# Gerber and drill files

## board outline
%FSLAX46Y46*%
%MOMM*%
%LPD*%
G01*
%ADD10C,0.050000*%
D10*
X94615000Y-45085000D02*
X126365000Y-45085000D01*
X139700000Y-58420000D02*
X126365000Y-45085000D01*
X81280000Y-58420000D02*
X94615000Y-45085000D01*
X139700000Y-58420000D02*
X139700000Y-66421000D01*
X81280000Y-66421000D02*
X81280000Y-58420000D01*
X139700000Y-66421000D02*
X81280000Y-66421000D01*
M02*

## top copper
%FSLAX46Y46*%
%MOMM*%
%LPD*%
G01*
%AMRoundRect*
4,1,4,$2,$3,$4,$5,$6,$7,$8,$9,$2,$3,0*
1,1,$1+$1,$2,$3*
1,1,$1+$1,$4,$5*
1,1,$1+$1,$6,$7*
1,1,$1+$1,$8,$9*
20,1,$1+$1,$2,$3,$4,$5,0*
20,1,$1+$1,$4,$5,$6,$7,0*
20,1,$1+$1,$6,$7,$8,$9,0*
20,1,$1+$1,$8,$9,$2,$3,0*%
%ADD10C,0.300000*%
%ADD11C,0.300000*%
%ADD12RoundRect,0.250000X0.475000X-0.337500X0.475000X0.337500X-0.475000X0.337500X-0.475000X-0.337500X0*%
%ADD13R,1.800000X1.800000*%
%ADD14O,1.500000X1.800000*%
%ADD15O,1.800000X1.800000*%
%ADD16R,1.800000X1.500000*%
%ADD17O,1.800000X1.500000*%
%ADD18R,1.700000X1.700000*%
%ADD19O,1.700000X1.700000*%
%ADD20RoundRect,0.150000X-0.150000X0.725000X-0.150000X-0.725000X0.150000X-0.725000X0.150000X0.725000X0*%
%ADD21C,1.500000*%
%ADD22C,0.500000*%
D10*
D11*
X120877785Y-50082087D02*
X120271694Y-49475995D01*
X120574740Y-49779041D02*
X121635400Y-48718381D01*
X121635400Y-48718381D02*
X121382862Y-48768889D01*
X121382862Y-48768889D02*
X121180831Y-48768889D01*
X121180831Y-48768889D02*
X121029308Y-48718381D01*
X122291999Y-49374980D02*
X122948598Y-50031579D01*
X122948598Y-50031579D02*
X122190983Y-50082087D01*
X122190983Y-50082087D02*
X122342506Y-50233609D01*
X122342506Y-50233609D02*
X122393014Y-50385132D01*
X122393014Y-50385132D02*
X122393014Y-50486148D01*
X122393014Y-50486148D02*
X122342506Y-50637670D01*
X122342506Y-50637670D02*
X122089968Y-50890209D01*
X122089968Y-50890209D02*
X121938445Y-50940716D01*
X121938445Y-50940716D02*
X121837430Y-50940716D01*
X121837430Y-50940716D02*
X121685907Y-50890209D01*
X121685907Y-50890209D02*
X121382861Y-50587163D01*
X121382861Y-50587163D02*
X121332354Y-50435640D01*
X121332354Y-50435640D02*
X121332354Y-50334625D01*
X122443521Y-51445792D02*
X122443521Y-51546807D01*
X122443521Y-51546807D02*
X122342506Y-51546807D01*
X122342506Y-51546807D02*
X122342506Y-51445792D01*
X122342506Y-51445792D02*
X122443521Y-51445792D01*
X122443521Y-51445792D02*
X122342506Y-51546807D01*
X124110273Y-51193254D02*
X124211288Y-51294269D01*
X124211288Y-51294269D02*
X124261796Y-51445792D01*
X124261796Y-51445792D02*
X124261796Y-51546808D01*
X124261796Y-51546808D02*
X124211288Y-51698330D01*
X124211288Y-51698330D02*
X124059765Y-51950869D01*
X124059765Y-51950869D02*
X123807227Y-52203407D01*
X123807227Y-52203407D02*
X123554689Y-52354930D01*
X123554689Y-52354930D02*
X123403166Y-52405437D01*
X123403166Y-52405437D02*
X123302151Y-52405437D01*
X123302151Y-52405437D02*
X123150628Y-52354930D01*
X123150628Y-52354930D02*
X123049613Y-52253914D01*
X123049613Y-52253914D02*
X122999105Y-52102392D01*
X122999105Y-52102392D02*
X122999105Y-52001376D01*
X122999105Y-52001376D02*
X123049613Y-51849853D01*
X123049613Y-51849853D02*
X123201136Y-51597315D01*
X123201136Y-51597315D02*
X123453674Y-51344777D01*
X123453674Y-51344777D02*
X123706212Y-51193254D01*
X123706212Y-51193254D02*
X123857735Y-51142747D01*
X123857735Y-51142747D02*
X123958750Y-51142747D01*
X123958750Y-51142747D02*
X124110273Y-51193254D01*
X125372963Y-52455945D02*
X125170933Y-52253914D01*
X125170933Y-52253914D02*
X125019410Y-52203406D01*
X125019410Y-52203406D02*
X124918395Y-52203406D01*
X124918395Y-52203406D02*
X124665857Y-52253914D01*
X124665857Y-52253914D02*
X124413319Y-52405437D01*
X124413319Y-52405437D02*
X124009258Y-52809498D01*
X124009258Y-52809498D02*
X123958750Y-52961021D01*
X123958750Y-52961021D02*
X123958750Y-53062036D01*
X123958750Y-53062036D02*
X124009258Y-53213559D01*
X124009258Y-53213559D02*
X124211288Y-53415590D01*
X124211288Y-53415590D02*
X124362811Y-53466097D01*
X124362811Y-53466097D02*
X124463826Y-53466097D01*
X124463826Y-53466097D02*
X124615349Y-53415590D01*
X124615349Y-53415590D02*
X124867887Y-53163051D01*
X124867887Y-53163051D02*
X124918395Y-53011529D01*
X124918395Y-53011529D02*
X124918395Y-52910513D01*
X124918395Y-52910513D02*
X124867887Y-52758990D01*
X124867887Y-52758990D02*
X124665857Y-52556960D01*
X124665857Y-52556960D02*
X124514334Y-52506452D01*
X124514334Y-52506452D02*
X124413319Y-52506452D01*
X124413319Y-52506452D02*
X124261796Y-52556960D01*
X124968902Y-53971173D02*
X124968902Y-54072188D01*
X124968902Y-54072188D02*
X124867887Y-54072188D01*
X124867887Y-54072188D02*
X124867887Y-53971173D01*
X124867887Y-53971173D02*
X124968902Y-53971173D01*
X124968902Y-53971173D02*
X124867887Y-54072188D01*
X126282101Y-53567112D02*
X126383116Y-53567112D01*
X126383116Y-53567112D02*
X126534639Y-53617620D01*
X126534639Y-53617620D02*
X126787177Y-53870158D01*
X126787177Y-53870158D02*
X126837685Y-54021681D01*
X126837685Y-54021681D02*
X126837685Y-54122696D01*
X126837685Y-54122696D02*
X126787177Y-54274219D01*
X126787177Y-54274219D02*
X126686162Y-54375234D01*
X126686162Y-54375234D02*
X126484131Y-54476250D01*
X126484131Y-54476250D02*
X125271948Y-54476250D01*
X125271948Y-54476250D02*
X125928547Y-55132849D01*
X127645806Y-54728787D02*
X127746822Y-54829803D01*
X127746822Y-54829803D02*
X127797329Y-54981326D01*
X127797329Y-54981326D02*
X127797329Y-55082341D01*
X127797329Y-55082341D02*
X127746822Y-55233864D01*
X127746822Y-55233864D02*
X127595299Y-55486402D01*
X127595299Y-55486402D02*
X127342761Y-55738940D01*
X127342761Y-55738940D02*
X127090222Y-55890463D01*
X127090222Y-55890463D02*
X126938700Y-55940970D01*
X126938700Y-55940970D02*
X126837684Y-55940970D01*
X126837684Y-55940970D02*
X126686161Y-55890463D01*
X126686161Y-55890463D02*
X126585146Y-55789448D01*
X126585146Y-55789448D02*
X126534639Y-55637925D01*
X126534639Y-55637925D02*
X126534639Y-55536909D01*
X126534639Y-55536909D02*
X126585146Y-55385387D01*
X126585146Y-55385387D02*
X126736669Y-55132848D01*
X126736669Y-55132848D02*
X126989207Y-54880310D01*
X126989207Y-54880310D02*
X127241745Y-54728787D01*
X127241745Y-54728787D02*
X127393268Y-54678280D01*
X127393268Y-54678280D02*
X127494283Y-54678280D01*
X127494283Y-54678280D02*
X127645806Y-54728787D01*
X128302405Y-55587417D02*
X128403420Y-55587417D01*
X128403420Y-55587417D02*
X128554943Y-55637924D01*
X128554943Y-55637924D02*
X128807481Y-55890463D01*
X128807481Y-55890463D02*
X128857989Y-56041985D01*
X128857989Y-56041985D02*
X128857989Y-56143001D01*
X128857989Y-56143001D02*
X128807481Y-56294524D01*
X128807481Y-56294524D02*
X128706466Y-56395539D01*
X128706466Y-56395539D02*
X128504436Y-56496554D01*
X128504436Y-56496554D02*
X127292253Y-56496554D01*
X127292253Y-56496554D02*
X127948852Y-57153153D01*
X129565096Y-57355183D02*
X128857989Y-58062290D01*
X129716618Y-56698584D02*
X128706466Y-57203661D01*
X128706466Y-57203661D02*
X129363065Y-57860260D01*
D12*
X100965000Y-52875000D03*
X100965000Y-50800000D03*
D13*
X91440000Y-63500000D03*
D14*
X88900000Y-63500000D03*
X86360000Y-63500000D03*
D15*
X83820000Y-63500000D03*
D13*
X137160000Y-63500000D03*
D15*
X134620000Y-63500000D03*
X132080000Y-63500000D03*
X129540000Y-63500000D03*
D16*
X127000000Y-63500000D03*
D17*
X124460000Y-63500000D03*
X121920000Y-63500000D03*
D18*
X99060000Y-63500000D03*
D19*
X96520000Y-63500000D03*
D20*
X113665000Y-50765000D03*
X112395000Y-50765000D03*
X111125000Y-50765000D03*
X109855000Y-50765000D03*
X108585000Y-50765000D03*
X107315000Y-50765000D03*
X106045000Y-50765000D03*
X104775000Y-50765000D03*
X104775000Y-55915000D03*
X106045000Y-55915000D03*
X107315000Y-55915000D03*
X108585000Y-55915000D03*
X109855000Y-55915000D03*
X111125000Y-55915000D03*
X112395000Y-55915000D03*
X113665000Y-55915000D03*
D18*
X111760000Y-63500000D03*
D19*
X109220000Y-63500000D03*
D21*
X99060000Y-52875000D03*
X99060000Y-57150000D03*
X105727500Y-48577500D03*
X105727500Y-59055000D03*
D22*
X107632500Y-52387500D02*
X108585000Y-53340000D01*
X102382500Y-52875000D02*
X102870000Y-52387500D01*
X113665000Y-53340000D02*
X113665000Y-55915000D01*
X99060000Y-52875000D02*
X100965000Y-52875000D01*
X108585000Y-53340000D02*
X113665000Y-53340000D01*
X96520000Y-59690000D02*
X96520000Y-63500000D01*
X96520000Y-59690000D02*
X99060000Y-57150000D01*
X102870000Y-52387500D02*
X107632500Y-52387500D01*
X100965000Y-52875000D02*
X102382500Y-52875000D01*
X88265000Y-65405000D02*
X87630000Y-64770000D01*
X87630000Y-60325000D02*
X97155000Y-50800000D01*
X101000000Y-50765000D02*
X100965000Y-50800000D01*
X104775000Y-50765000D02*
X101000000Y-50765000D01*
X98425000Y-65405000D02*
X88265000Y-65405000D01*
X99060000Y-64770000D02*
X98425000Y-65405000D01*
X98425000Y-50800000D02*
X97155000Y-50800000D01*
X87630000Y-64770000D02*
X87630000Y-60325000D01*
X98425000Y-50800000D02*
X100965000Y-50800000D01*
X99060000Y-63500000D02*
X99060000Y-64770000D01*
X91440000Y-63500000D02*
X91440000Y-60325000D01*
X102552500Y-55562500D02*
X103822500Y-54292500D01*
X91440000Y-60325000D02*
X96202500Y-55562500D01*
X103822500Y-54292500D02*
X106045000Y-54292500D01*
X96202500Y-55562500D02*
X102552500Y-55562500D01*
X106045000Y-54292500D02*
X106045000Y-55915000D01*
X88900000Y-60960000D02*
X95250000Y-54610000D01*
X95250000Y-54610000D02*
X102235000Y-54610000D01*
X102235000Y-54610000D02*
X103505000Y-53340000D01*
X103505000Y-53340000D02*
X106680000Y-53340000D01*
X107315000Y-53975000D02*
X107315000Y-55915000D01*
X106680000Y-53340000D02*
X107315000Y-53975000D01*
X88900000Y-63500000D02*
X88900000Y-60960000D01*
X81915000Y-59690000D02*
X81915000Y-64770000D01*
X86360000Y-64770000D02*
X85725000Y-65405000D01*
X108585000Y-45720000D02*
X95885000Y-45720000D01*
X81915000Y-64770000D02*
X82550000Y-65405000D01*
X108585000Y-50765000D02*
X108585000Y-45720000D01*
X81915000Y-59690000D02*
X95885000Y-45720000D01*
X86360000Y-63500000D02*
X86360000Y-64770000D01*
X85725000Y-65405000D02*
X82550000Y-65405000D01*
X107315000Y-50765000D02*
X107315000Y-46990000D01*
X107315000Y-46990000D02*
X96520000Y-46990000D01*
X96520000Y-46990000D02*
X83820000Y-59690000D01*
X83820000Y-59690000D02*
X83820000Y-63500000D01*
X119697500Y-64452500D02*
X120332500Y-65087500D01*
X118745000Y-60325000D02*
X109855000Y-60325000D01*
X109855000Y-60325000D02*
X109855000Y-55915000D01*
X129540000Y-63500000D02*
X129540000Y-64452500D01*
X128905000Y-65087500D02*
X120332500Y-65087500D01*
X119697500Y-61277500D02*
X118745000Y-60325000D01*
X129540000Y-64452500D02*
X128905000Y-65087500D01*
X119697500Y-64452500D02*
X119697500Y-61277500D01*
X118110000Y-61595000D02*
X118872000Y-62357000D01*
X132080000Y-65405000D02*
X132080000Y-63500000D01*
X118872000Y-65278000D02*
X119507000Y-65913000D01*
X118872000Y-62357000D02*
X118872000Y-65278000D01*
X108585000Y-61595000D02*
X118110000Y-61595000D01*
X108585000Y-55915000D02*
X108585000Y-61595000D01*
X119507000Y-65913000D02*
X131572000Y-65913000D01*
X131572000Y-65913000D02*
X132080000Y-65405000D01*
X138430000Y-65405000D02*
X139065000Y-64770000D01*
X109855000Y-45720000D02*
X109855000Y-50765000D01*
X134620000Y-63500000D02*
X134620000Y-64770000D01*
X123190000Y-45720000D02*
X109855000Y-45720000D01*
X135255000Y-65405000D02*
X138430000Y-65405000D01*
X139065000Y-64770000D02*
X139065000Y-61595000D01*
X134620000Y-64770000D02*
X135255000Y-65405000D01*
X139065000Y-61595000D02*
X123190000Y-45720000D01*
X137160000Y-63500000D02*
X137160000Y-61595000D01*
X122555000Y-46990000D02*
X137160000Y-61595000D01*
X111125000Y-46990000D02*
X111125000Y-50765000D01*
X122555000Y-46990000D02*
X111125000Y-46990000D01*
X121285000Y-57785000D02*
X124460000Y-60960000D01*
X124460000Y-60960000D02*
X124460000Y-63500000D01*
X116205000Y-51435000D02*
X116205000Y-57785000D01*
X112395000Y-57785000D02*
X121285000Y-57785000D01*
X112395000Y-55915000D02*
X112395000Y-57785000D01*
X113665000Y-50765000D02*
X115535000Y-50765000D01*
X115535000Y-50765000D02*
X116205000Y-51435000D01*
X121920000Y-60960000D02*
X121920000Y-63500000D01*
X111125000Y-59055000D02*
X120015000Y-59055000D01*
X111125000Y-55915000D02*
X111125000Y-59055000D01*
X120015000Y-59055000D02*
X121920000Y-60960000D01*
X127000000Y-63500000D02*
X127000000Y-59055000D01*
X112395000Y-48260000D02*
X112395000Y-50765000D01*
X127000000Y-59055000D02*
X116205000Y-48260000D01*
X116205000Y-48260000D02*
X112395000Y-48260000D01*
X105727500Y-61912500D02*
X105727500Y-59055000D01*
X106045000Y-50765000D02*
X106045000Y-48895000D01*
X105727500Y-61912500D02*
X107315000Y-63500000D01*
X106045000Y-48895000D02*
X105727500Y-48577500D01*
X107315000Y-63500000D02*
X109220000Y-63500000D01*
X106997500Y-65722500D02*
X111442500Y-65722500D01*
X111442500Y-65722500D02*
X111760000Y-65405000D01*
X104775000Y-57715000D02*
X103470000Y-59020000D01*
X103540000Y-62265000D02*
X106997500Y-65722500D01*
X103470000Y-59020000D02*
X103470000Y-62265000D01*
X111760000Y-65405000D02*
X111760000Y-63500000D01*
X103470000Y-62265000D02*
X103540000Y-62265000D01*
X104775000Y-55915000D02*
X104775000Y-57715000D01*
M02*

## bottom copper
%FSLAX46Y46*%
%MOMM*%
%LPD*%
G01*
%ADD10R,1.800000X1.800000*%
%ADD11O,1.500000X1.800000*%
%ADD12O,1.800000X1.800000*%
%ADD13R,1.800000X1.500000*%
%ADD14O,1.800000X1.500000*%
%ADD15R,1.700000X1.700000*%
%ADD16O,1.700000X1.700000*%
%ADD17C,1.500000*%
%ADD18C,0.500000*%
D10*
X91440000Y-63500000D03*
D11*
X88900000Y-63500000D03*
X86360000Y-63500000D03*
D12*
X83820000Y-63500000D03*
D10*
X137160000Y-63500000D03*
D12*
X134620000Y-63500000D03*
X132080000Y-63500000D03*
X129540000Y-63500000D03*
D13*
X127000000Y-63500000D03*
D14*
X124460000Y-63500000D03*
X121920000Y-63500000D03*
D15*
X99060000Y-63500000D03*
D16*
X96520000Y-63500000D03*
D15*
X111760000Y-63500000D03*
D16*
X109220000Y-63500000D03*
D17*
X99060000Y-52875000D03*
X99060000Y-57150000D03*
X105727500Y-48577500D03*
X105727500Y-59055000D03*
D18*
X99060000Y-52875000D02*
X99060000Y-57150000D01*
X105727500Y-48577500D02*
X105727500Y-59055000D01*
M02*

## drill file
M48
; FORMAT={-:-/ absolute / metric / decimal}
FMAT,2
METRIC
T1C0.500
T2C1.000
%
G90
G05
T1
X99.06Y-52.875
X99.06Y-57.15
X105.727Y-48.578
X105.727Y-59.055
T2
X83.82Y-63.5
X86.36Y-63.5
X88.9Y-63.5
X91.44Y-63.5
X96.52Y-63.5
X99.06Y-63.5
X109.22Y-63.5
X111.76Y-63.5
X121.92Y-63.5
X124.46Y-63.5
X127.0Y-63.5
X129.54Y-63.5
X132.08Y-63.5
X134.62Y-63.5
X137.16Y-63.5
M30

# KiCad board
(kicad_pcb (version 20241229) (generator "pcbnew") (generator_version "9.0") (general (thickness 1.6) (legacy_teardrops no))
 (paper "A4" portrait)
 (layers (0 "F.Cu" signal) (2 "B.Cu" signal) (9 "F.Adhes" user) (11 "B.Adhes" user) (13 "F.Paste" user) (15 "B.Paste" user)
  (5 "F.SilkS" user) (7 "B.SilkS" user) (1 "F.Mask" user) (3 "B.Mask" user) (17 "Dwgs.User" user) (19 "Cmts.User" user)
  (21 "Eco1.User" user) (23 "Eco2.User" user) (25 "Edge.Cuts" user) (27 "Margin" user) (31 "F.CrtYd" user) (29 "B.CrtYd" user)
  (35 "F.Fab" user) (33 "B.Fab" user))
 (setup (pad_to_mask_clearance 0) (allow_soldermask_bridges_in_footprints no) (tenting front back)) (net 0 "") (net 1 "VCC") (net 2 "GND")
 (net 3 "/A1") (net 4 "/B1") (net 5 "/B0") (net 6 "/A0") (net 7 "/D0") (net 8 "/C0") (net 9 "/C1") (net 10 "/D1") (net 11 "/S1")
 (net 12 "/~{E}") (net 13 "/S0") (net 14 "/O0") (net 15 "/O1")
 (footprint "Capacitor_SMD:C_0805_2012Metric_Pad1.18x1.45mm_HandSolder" (layer "F.Cu") (at 100.965 51.8375 90)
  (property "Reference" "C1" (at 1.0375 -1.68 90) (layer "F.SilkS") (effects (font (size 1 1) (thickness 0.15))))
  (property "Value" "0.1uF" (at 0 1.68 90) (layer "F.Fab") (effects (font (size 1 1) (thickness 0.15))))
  (pad "1" smd roundrect (at -1.0375 0 90) (size 1.175 1.45) (layers "F.Cu" "F.Mask" "F.Paste") (roundrect_rratio 0.2127659574)
   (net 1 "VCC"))
  (pad "2" smd roundrect (at 1.0375 0 90) (size 1.175 1.45) (layers "F.Cu" "F.Mask" "F.Paste") (roundrect_rratio 0.2127659574) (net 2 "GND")))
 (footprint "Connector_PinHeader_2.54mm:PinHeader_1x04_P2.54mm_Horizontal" (layer "F.Cu") (at 91.44 63.5 -90)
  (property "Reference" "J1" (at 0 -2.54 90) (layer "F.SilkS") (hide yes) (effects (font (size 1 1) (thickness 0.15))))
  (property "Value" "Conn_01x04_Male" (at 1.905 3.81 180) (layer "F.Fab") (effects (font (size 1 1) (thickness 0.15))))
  (pad "1" thru_hole rect (at 0 0 270) (size 1.8 1.8) (drill 1) (layers "*.Cu" "*.Mask") (remove_unused_layers no) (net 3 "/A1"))
  (pad "2" thru_hole oval (at 0 2.54 270) (size 1.8 1.5) (drill 1) (layers "*.Cu" "*.Mask") (remove_unused_layers no) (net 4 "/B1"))
  (pad "3" thru_hole oval (at 0 5.08 270) (size 1.8 1.5) (drill 1) (layers "*.Cu" "*.Mask") (remove_unused_layers no) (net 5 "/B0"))
  (pad "4" thru_hole oval (at 0 7.62 270) (size 1.8 1.8) (drill 1) (layers "*.Cu" "*.Mask") (remove_unused_layers no) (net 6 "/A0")))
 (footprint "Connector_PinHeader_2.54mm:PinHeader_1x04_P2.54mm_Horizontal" (layer "F.Cu") (at 137.16 63.5 -90)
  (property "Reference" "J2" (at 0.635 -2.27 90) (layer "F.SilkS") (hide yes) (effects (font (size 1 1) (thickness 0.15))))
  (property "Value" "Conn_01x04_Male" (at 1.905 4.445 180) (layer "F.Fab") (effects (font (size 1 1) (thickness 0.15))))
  (pad "1" thru_hole rect (at 0 0 270) (size 1.8 1.8) (drill 1) (layers "*.Cu" "*.Mask") (remove_unused_layers no) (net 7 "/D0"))
  (pad "2" thru_hole oval (at 0 2.54 270) (size 1.8 1.8) (drill 1) (layers "*.Cu" "*.Mask") (remove_unused_layers no) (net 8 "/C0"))
  (pad "3" thru_hole oval (at 0 5.08 270) (size 1.8 1.8) (drill 1) (layers "*.Cu" "*.Mask") (remove_unused_layers no) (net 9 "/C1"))
  (pad "4" thru_hole oval (at 0 7.62 270) (size 1.8 1.8) (drill 1) (layers "*.Cu" "*.Mask") (remove_unused_layers no) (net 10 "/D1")))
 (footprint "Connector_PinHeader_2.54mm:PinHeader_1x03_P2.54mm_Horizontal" (layer "F.Cu") (at 127 63.5 -90)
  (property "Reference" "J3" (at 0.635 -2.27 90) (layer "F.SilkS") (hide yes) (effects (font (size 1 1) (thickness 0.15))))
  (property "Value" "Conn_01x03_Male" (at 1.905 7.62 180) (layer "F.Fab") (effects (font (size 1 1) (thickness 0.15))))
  (pad "1" thru_hole rect (at 0 0 270) (size 1.5 1.8) (drill 1) (layers "*.Cu" "*.Mask") (remove_unused_layers no) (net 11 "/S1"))
  (pad "2" thru_hole oval (at 0 2.54 270) (size 1.5 1.8) (drill 1) (layers "*.Cu" "*.Mask") (remove_unused_layers no) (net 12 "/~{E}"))
  (pad "3" thru_hole oval (at 0 5.08 270) (size 1.5 1.8) (drill 1) (layers "*.Cu" "*.Mask") (remove_unused_layers no) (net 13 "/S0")))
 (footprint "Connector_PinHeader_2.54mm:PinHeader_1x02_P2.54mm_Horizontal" (layer "F.Cu") (at 99.06 63.5 -90)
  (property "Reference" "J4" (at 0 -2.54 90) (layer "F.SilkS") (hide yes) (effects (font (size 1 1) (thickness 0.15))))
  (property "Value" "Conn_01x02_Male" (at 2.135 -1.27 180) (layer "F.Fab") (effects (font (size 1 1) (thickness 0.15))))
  (pad "1" thru_hole rect (at 0 0 270) (size 1.7 1.7) (drill 1) (layers "*.Cu" "*.Mask") (remove_unused_layers no) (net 2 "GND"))
  (pad "2" thru_hole oval (at 0 2.54 270) (size 1.7 1.7) (drill 1) (layers "*.Cu" "*.Mask") (remove_unused_layers no) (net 1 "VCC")))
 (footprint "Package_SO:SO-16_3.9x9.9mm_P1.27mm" (layer "F.Cu") (at 109.22 53.34 -90)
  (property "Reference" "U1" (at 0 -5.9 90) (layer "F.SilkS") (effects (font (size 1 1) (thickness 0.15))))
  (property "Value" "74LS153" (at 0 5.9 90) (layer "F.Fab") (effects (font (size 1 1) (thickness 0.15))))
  (pad "1" smd roundrect (at -2.575 -4.445 270) (size 1.75 0.6) (layers "F.Cu" "F.Mask" "F.Paste") (roundrect_rratio 0.25) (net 12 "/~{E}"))
  (pad "2" smd roundrect (at -2.575 -3.175 270) (size 1.75 0.6) (layers "F.Cu" "F.Mask" "F.Paste") (roundrect_rratio 0.25) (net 11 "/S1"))
  (pad "3" smd roundrect (at -2.575 -1.905 270) (size 1.75 0.6) (layers "F.Cu" "F.Mask" "F.Paste") (roundrect_rratio 0.25) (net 7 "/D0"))
  (pad "4" smd roundrect (at -2.575 -0.635 270) (size 1.75 0.6) (layers "F.Cu" "F.Mask" "F.Paste") (roundrect_rratio 0.25) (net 8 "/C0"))
  (pad "5" smd roundrect (at -2.575 0.635 270) (size 1.75 0.6) (layers "F.Cu" "F.Mask" "F.Paste") (roundrect_rratio 0.25) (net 5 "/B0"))
  (pad "6" smd roundrect (at -2.575 1.905 270) (size 1.75 0.6) (layers "F.Cu" "F.Mask" "F.Paste") (roundrect_rratio 0.25) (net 6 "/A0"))
  (pad "7" smd roundrect (at -2.575 3.175 270) (size 1.75 0.6) (layers "F.Cu" "F.Mask" "F.Paste") (roundrect_rratio 0.25) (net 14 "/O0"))
  (pad "8" smd roundrect (at -2.575 4.445 270) (size 1.75 0.6) (layers "F.Cu" "F.Mask" "F.Paste") (roundrect_rratio 0.25) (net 2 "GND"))
  (pad "9" smd roundrect (at 2.575 4.445 270) (size 1.75 0.6) (layers "F.Cu" "F.Mask" "F.Paste") (roundrect_rratio 0.25) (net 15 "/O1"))
  (pad "10" smd roundrect (at 2.575 3.175 270) (size 1.75 0.6) (layers "F.Cu" "F.Mask" "F.Paste") (roundrect_rratio 0.25) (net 3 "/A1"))
  (pad "11" smd roundrect (at 2.575 1.905 270) (size 1.75 0.6) (layers "F.Cu" "F.Mask" "F.Paste") (roundrect_rratio 0.25) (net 4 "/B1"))
  (pad "12" smd roundrect (at 2.575 0.635 270) (size 1.75 0.6) (layers "F.Cu" "F.Mask" "F.Paste") (roundrect_rratio 0.25) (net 9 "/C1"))
  (pad "13" smd roundrect (at 2.575 -0.635 270) (size 1.75 0.6) (layers "F.Cu" "F.Mask" "F.Paste") (roundrect_rratio 0.25) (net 10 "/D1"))
  (pad "14" smd roundrect (at 2.575 -1.905 270) (size 1.75 0.6) (layers "F.Cu" "F.Mask" "F.Paste") (roundrect_rratio 0.25) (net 13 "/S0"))
  (pad "15" smd roundrect (at 2.575 -3.175 270) (size 1.75 0.6) (layers "F.Cu" "F.Mask" "F.Paste") (roundrect_rratio 0.25) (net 12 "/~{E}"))
  (pad "16" smd roundrect (at 2.575 -4.445 270) (size 1.75 0.6) (layers "F.Cu" "F.Mask" "F.Paste") (roundrect_rratio 0.25) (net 1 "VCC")))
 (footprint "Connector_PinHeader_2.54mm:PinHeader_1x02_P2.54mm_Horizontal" (layer "F.Cu") (at 111.76 63.5 -90)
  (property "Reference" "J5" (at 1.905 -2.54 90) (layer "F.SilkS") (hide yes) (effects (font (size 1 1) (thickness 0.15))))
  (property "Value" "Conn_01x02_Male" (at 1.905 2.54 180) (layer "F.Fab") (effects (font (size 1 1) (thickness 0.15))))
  (pad "1" thru_hole rect (at 0 0 270) (size 1.7 1.7) (drill 1) (layers "*.Cu" "*.Mask") (remove_unused_layers no) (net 15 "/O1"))
  (pad "2" thru_hole oval (at 0 2.54 270) (size 1.7 1.7) (drill 1) (layers "*.Cu" "*.Mask") (remove_unused_layers no) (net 14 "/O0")))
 (gr_line (start 94.615 45.085) (end 126.365 45.085) (stroke (width 0.05) (type solid)) (layer "Edge.Cuts"))
 (gr_line (start 139.7 58.42) (end 126.365 45.085) (stroke (width 0.05) (type solid)) (layer "Edge.Cuts"))
 (gr_line (start 81.28 58.42) (end 94.615 45.085) (stroke (width 0.05) (type solid)) (layer "Edge.Cuts"))
 (gr_line (start 139.7 58.42) (end 139.7 66.421) (stroke (width 0.05) (type solid)) (layer "Edge.Cuts"))
 (gr_line (start 81.28 66.421) (end 81.28 58.42) (stroke (width 0.05) (type solid)) (layer "Edge.Cuts"))
 (gr_line (start 139.7 66.421) (end 81.28 66.421) (stroke (width 0.05) (type solid)) (layer "Edge.Cuts"))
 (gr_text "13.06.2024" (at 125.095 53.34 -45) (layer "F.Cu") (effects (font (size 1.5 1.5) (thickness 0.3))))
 (segment (start 107.6325 52.3875) (end 108.585 53.34) (width 0.5) (layer "F.Cu") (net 1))
 (segment (start 102.3825 52.875) (end 102.87 52.3875) (width 0.5) (layer "F.Cu") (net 1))
 (segment (start 113.665 53.34) (end 113.665 55.915) (width 0.5) (layer "F.Cu") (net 1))
 (segment (start 99.06 52.875) (end 100.965 52.875) (width 0.5) (layer "F.Cu") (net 1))
 (segment (start 108.585 53.34) (end 113.665 53.34) (width 0.5) (layer "F.Cu") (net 1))
 (segment (start 96.52 59.69) (end 96.52 63.5) (width 0.5) (layer "F.Cu") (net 1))
 (segment (start 96.52 59.69) (end 99.06 57.15) (width 0.5) (layer "F.Cu") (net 1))
 (segment (start 102.87 52.3875) (end 107.6325 52.3875) (width 0.5) (layer "F.Cu") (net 1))
 (segment (start 100.965 52.875) (end 102.3825 52.875) (width 0.5) (layer "F.Cu") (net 1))
 (via (at 99.06 52.875) (size 1.5) (drill 0.5) (layers "F.Cu" "B.Cu") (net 1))
 (via (at 99.06 57.15) (size 1.5) (drill 0.5) (layers "F.Cu" "B.Cu") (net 1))
 (segment (start 99.06 52.875) (end 99.06 57.15) (width 0.5) (layer "B.Cu") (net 1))
 (segment (start 88.265 65.405) (end 87.63 64.77) (width 0.5) (layer "F.Cu") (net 2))
 (segment (start 87.63 60.325) (end 97.155 50.8) (width 0.5) (layer "F.Cu") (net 2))
 (segment (start 101 50.765) (end 100.965 50.8) (width 0.5) (layer "F.Cu") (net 2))
 (segment (start 104.775 50.765) (end 101 50.765) (width 0.5) (layer "F.Cu") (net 2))
 (segment (start 98.425 65.405) (end 88.265 65.405) (width 0.5) (layer "F.Cu") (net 2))
 (segment (start 99.06 64.77) (end 98.425 65.405) (width 0.5) (layer "F.Cu") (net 2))
 (segment (start 98.425 50.8) (end 97.155 50.8) (width 0.5) (layer "F.Cu") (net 2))
 (segment (start 87.63 64.77) (end 87.63 60.325) (width 0.5) (layer "F.Cu") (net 2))
 (segment (start 98.425 50.8) (end 100.965 50.8) (width 0.5) (layer "F.Cu") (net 2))
 (segment (start 99.06 63.5) (end 99.06 64.77) (width 0.5) (layer "F.Cu") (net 2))
 (segment (start 91.44 63.5) (end 91.44 60.325) (width 0.5) (layer "F.Cu") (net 3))
 (segment (start 102.5525 55.5625) (end 103.8225 54.2925) (width 0.5) (layer "F.Cu") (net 3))
 (segment (start 91.44 60.325) (end 96.2025 55.5625) (width 0.5) (layer "F.Cu") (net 3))
 (segment (start 103.8225 54.2925) (end 106.045 54.2925) (width 0.5) (layer "F.Cu") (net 3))
 (segment (start 96.2025 55.5625) (end 102.5525 55.5625) (width 0.5) (layer "F.Cu") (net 3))
 (segment (start 106.045 54.2925) (end 106.045 55.915) (width 0.5) (layer "F.Cu") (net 3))
 (segment (start 88.9 60.96) (end 95.25 54.61) (width 0.5) (layer "F.Cu") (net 4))
 (segment (start 95.25 54.61) (end 102.235 54.61) (width 0.5) (layer "F.Cu") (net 4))
 (segment (start 102.235 54.61) (end 103.505 53.34) (width 0.5) (layer "F.Cu") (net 4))
 (segment (start 103.505 53.34) (end 106.68 53.34) (width 0.5) (layer "F.Cu") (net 4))
 (segment (start 107.315 53.975) (end 107.315 55.915) (width 0.5) (layer "F.Cu") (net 4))
 (segment (start 106.68 53.34) (end 107.315 53.975) (width 0.5) (layer "F.Cu") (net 4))
 (segment (start 88.9 63.5) (end 88.9 60.96) (width 0.5) (layer "F.Cu") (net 4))
 (segment (start 81.915 59.69) (end 81.915 64.77) (width 0.5) (layer "F.Cu") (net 5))
 (segment (start 86.36 64.77) (end 85.725 65.405) (width 0.5) (layer "F.Cu") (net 5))
 (segment (start 108.585 45.72) (end 95.885 45.72) (width 0.5) (layer "F.Cu") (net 5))
 (segment (start 81.915 64.77) (end 82.55 65.405) (width 0.5) (layer "F.Cu") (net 5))
 (segment (start 108.585 50.765) (end 108.585 45.72) (width 0.5) (layer "F.Cu") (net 5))
 (segment (start 81.915 59.69) (end 95.885 45.72) (width 0.5) (layer "F.Cu") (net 5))
 (segment (start 86.36 63.5) (end 86.36 64.77) (width 0.5) (layer "F.Cu") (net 5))
 (segment (start 85.725 65.405) (end 82.55 65.405) (width 0.5) (layer "F.Cu") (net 5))
 (segment (start 107.315 50.765) (end 107.315 46.99) (width 0.5) (layer "F.Cu") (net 6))
 (segment (start 107.315 46.99) (end 96.52 46.99) (width 0.5) (layer "F.Cu") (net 6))
 (segment (start 96.52 46.99) (end 83.82 59.69) (width 0.5) (layer "F.Cu") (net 6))
 (segment (start 83.82 59.69) (end 83.82 63.5) (width 0.5) (layer "F.Cu") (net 6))
 (segment (start 119.6975 64.4525) (end 120.3325 65.0875) (width 0.5) (layer "F.Cu") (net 10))
 (segment (start 118.745 60.325) (end 109.855 60.325) (width 0.5) (layer "F.Cu") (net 10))
 (segment (start 109.855 60.325) (end 109.855 55.915) (width 0.5) (layer "F.Cu") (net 10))
 (segment (start 129.54 63.5) (end 129.54 64.4525) (width 0.5) (layer "F.Cu") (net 10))
 (segment (start 128.905 65.0875) (end 120.3325 65.0875) (width 0.5) (layer "F.Cu") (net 10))
 (segment (start 119.6975 61.2775) (end 118.745 60.325) (width 0.5) (layer "F.Cu") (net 10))
 (segment (start 129.54 64.4525) (end 128.905 65.0875) (width 0.5) (layer "F.Cu") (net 10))
 (segment (start 119.6975 64.4525) (end 119.6975 61.2775) (width 0.5) (layer "F.Cu") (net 10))
 (segment (start 118.11 61.595) (end 118.872 62.357) (width 0.5) (layer "F.Cu") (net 9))
 (segment (start 132.08 65.405) (end 132.08 63.5) (width 0.5) (layer "F.Cu") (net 9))
 (segment (start 118.872 65.278) (end 119.507 65.913) (width 0.5) (layer "F.Cu") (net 9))
 (segment (start 118.872 62.357) (end 118.872 65.278) (width 0.5) (layer "F.Cu") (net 9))
 (segment (start 108.585 61.595) (end 118.11 61.595) (width 0.5) (layer "F.Cu") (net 9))
 (segment (start 108.585 55.915) (end 108.585 61.595) (width 0.5) (layer "F.Cu") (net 9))
 (segment (start 119.507 65.913) (end 131.572 65.913) (width 0.5) (layer "F.Cu") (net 9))
 (segment (start 131.572 65.913) (end 132.08 65.405) (width 0.5) (layer "F.Cu") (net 9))
 (segment (start 138.43 65.405) (end 139.065 64.77) (width 0.5) (layer "F.Cu") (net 8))
 (segment (start 109.855 45.72) (end 109.855 50.765) (width 0.5) (layer "F.Cu") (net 8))
 (segment (start 134.62 63.5) (end 134.62 64.77) (width 0.5) (layer "F.Cu") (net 8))
 (segment (start 123.19 45.72) (end 109.855 45.72) (width 0.5) (layer "F.Cu") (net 8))
 (segment (start 135.255 65.405) (end 138.43 65.405) (width 0.5) (layer "F.Cu") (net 8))
 (segment (start 139.065 64.77) (end 139.065 61.595) (width 0.5) (layer "F.Cu") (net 8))
 (segment (start 134.62 64.77) (end 135.255 65.405) (width 0.5) (layer "F.Cu") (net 8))
 (segment (start 139.065 61.595) (end 123.19 45.72) (width 0.5) (layer "F.Cu") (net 8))
 (segment (start 137.16 63.5) (end 137.16 61.595) (width 0.5) (layer "F.Cu") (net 7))
 (segment (start 122.555 46.99) (end 137.16 61.595) (width 0.5) (layer "F.Cu") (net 7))
 (segment (start 111.125 46.99) (end 111.125 50.765) (width 0.5) (layer "F.Cu") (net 7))
 (segment (start 122.555 46.99) (end 111.125 46.99) (width 0.5) (layer "F.Cu") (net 7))
 (segment (start 121.285 57.785) (end 124.46 60.96) (width 0.5) (layer "F.Cu") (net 12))
 (segment (start 124.46 60.96) (end 124.46 63.5) (width 0.5) (layer "F.Cu") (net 12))
 (segment (start 116.205 51.435) (end 116.205 57.785) (width 0.5) (layer "F.Cu") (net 12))
 (segment (start 112.395 57.785) (end 121.285 57.785) (width 0.5) (layer "F.Cu") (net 12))
 (segment (start 112.395 55.915) (end 112.395 57.785) (width 0.5) (layer "F.Cu") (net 12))
 (segment (start 113.665 50.765) (end 115.535 50.765) (width 0.5) (layer "F.Cu") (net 12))
 (segment (start 115.535 50.765) (end 116.205 51.435) (width 0.5) (layer "F.Cu") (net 12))
 (segment (start 121.92 60.96) (end 121.92 63.5) (width 0.5) (layer "F.Cu") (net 13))
 (segment (start 111.125 59.055) (end 120.015 59.055) (width 0.5) (layer "F.Cu") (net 13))
 (segment (start 111.125 55.915) (end 111.125 59.055) (width 0.5) (layer "F.Cu") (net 13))
 (segment (start 120.015 59.055) (end 121.92 60.96) (width 0.5) (layer "F.Cu") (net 13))
 (segment (start 127 63.5) (end 127 59.055) (width 0.5) (layer "F.Cu") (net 11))
 (segment (start 112.395 48.26) (end 112.395 50.765) (width 0.5) (layer "F.Cu") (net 11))
 (segment (start 127 59.055) (end 116.205 48.26) (width 0.5) (layer "F.Cu") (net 11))
 (segment (start 116.205 48.26) (end 112.395 48.26) (width 0.5) (layer "F.Cu") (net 11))
 (segment (start 105.7275 61.9125) (end 105.7275 59.055) (width 0.5) (layer "F.Cu") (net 14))
 (segment (start 106.045 50.765) (end 106.045 48.895) (width 0.5) (layer "F.Cu") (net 14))
 (segment (start 105.7275 61.9125) (end 107.315 63.5) (width 0.5) (layer "F.Cu") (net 14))
 (segment (start 106.045 48.895) (end 105.7275 48.5775) (width 0.5) (layer "F.Cu") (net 14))
 (segment (start 107.315 63.5) (end 109.22 63.5) (width 0.5) (layer "F.Cu") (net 14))
 (via (at 105.7275 48.5775) (size 1.5) (drill 0.5) (layers "F.Cu" "B.Cu") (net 14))
 (via (at 105.7275 59.055) (size 1.5) (drill 0.5) (layers "F.Cu" "B.Cu") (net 14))
 (segment (start 105.7275 48.5775) (end 105.7275 59.055) (width 0.5) (layer "B.Cu") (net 14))
 (segment (start 106.9975 65.7225) (end 111.4425 65.7225) (width 0.5) (layer "F.Cu") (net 15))
 (segment (start 111.4425 65.7225) (end 111.76 65.405) (width 0.5) (layer "F.Cu") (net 15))
 (segment (start 104.775 57.715) (end 103.47 59.02) (width 0.5) (layer "F.Cu") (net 15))
 (segment (start 103.54 62.265) (end 106.9975 65.7225) (width 0.5) (layer "F.Cu") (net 15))
 (segment (start 103.47 59.02) (end 103.47 62.265) (width 0.5) (layer "F.Cu") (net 15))
 (segment (start 111.76 65.405) (end 111.76 63.5) (width 0.5) (layer "F.Cu") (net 15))
 (segment (start 103.47 62.265) (end 103.54 62.265) (width 0.5) (layer "F.Cu") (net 15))
 (segment (start 104.775 55.915) (end 104.775 57.715) (width 0.5) (layer "F.Cu") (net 15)))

